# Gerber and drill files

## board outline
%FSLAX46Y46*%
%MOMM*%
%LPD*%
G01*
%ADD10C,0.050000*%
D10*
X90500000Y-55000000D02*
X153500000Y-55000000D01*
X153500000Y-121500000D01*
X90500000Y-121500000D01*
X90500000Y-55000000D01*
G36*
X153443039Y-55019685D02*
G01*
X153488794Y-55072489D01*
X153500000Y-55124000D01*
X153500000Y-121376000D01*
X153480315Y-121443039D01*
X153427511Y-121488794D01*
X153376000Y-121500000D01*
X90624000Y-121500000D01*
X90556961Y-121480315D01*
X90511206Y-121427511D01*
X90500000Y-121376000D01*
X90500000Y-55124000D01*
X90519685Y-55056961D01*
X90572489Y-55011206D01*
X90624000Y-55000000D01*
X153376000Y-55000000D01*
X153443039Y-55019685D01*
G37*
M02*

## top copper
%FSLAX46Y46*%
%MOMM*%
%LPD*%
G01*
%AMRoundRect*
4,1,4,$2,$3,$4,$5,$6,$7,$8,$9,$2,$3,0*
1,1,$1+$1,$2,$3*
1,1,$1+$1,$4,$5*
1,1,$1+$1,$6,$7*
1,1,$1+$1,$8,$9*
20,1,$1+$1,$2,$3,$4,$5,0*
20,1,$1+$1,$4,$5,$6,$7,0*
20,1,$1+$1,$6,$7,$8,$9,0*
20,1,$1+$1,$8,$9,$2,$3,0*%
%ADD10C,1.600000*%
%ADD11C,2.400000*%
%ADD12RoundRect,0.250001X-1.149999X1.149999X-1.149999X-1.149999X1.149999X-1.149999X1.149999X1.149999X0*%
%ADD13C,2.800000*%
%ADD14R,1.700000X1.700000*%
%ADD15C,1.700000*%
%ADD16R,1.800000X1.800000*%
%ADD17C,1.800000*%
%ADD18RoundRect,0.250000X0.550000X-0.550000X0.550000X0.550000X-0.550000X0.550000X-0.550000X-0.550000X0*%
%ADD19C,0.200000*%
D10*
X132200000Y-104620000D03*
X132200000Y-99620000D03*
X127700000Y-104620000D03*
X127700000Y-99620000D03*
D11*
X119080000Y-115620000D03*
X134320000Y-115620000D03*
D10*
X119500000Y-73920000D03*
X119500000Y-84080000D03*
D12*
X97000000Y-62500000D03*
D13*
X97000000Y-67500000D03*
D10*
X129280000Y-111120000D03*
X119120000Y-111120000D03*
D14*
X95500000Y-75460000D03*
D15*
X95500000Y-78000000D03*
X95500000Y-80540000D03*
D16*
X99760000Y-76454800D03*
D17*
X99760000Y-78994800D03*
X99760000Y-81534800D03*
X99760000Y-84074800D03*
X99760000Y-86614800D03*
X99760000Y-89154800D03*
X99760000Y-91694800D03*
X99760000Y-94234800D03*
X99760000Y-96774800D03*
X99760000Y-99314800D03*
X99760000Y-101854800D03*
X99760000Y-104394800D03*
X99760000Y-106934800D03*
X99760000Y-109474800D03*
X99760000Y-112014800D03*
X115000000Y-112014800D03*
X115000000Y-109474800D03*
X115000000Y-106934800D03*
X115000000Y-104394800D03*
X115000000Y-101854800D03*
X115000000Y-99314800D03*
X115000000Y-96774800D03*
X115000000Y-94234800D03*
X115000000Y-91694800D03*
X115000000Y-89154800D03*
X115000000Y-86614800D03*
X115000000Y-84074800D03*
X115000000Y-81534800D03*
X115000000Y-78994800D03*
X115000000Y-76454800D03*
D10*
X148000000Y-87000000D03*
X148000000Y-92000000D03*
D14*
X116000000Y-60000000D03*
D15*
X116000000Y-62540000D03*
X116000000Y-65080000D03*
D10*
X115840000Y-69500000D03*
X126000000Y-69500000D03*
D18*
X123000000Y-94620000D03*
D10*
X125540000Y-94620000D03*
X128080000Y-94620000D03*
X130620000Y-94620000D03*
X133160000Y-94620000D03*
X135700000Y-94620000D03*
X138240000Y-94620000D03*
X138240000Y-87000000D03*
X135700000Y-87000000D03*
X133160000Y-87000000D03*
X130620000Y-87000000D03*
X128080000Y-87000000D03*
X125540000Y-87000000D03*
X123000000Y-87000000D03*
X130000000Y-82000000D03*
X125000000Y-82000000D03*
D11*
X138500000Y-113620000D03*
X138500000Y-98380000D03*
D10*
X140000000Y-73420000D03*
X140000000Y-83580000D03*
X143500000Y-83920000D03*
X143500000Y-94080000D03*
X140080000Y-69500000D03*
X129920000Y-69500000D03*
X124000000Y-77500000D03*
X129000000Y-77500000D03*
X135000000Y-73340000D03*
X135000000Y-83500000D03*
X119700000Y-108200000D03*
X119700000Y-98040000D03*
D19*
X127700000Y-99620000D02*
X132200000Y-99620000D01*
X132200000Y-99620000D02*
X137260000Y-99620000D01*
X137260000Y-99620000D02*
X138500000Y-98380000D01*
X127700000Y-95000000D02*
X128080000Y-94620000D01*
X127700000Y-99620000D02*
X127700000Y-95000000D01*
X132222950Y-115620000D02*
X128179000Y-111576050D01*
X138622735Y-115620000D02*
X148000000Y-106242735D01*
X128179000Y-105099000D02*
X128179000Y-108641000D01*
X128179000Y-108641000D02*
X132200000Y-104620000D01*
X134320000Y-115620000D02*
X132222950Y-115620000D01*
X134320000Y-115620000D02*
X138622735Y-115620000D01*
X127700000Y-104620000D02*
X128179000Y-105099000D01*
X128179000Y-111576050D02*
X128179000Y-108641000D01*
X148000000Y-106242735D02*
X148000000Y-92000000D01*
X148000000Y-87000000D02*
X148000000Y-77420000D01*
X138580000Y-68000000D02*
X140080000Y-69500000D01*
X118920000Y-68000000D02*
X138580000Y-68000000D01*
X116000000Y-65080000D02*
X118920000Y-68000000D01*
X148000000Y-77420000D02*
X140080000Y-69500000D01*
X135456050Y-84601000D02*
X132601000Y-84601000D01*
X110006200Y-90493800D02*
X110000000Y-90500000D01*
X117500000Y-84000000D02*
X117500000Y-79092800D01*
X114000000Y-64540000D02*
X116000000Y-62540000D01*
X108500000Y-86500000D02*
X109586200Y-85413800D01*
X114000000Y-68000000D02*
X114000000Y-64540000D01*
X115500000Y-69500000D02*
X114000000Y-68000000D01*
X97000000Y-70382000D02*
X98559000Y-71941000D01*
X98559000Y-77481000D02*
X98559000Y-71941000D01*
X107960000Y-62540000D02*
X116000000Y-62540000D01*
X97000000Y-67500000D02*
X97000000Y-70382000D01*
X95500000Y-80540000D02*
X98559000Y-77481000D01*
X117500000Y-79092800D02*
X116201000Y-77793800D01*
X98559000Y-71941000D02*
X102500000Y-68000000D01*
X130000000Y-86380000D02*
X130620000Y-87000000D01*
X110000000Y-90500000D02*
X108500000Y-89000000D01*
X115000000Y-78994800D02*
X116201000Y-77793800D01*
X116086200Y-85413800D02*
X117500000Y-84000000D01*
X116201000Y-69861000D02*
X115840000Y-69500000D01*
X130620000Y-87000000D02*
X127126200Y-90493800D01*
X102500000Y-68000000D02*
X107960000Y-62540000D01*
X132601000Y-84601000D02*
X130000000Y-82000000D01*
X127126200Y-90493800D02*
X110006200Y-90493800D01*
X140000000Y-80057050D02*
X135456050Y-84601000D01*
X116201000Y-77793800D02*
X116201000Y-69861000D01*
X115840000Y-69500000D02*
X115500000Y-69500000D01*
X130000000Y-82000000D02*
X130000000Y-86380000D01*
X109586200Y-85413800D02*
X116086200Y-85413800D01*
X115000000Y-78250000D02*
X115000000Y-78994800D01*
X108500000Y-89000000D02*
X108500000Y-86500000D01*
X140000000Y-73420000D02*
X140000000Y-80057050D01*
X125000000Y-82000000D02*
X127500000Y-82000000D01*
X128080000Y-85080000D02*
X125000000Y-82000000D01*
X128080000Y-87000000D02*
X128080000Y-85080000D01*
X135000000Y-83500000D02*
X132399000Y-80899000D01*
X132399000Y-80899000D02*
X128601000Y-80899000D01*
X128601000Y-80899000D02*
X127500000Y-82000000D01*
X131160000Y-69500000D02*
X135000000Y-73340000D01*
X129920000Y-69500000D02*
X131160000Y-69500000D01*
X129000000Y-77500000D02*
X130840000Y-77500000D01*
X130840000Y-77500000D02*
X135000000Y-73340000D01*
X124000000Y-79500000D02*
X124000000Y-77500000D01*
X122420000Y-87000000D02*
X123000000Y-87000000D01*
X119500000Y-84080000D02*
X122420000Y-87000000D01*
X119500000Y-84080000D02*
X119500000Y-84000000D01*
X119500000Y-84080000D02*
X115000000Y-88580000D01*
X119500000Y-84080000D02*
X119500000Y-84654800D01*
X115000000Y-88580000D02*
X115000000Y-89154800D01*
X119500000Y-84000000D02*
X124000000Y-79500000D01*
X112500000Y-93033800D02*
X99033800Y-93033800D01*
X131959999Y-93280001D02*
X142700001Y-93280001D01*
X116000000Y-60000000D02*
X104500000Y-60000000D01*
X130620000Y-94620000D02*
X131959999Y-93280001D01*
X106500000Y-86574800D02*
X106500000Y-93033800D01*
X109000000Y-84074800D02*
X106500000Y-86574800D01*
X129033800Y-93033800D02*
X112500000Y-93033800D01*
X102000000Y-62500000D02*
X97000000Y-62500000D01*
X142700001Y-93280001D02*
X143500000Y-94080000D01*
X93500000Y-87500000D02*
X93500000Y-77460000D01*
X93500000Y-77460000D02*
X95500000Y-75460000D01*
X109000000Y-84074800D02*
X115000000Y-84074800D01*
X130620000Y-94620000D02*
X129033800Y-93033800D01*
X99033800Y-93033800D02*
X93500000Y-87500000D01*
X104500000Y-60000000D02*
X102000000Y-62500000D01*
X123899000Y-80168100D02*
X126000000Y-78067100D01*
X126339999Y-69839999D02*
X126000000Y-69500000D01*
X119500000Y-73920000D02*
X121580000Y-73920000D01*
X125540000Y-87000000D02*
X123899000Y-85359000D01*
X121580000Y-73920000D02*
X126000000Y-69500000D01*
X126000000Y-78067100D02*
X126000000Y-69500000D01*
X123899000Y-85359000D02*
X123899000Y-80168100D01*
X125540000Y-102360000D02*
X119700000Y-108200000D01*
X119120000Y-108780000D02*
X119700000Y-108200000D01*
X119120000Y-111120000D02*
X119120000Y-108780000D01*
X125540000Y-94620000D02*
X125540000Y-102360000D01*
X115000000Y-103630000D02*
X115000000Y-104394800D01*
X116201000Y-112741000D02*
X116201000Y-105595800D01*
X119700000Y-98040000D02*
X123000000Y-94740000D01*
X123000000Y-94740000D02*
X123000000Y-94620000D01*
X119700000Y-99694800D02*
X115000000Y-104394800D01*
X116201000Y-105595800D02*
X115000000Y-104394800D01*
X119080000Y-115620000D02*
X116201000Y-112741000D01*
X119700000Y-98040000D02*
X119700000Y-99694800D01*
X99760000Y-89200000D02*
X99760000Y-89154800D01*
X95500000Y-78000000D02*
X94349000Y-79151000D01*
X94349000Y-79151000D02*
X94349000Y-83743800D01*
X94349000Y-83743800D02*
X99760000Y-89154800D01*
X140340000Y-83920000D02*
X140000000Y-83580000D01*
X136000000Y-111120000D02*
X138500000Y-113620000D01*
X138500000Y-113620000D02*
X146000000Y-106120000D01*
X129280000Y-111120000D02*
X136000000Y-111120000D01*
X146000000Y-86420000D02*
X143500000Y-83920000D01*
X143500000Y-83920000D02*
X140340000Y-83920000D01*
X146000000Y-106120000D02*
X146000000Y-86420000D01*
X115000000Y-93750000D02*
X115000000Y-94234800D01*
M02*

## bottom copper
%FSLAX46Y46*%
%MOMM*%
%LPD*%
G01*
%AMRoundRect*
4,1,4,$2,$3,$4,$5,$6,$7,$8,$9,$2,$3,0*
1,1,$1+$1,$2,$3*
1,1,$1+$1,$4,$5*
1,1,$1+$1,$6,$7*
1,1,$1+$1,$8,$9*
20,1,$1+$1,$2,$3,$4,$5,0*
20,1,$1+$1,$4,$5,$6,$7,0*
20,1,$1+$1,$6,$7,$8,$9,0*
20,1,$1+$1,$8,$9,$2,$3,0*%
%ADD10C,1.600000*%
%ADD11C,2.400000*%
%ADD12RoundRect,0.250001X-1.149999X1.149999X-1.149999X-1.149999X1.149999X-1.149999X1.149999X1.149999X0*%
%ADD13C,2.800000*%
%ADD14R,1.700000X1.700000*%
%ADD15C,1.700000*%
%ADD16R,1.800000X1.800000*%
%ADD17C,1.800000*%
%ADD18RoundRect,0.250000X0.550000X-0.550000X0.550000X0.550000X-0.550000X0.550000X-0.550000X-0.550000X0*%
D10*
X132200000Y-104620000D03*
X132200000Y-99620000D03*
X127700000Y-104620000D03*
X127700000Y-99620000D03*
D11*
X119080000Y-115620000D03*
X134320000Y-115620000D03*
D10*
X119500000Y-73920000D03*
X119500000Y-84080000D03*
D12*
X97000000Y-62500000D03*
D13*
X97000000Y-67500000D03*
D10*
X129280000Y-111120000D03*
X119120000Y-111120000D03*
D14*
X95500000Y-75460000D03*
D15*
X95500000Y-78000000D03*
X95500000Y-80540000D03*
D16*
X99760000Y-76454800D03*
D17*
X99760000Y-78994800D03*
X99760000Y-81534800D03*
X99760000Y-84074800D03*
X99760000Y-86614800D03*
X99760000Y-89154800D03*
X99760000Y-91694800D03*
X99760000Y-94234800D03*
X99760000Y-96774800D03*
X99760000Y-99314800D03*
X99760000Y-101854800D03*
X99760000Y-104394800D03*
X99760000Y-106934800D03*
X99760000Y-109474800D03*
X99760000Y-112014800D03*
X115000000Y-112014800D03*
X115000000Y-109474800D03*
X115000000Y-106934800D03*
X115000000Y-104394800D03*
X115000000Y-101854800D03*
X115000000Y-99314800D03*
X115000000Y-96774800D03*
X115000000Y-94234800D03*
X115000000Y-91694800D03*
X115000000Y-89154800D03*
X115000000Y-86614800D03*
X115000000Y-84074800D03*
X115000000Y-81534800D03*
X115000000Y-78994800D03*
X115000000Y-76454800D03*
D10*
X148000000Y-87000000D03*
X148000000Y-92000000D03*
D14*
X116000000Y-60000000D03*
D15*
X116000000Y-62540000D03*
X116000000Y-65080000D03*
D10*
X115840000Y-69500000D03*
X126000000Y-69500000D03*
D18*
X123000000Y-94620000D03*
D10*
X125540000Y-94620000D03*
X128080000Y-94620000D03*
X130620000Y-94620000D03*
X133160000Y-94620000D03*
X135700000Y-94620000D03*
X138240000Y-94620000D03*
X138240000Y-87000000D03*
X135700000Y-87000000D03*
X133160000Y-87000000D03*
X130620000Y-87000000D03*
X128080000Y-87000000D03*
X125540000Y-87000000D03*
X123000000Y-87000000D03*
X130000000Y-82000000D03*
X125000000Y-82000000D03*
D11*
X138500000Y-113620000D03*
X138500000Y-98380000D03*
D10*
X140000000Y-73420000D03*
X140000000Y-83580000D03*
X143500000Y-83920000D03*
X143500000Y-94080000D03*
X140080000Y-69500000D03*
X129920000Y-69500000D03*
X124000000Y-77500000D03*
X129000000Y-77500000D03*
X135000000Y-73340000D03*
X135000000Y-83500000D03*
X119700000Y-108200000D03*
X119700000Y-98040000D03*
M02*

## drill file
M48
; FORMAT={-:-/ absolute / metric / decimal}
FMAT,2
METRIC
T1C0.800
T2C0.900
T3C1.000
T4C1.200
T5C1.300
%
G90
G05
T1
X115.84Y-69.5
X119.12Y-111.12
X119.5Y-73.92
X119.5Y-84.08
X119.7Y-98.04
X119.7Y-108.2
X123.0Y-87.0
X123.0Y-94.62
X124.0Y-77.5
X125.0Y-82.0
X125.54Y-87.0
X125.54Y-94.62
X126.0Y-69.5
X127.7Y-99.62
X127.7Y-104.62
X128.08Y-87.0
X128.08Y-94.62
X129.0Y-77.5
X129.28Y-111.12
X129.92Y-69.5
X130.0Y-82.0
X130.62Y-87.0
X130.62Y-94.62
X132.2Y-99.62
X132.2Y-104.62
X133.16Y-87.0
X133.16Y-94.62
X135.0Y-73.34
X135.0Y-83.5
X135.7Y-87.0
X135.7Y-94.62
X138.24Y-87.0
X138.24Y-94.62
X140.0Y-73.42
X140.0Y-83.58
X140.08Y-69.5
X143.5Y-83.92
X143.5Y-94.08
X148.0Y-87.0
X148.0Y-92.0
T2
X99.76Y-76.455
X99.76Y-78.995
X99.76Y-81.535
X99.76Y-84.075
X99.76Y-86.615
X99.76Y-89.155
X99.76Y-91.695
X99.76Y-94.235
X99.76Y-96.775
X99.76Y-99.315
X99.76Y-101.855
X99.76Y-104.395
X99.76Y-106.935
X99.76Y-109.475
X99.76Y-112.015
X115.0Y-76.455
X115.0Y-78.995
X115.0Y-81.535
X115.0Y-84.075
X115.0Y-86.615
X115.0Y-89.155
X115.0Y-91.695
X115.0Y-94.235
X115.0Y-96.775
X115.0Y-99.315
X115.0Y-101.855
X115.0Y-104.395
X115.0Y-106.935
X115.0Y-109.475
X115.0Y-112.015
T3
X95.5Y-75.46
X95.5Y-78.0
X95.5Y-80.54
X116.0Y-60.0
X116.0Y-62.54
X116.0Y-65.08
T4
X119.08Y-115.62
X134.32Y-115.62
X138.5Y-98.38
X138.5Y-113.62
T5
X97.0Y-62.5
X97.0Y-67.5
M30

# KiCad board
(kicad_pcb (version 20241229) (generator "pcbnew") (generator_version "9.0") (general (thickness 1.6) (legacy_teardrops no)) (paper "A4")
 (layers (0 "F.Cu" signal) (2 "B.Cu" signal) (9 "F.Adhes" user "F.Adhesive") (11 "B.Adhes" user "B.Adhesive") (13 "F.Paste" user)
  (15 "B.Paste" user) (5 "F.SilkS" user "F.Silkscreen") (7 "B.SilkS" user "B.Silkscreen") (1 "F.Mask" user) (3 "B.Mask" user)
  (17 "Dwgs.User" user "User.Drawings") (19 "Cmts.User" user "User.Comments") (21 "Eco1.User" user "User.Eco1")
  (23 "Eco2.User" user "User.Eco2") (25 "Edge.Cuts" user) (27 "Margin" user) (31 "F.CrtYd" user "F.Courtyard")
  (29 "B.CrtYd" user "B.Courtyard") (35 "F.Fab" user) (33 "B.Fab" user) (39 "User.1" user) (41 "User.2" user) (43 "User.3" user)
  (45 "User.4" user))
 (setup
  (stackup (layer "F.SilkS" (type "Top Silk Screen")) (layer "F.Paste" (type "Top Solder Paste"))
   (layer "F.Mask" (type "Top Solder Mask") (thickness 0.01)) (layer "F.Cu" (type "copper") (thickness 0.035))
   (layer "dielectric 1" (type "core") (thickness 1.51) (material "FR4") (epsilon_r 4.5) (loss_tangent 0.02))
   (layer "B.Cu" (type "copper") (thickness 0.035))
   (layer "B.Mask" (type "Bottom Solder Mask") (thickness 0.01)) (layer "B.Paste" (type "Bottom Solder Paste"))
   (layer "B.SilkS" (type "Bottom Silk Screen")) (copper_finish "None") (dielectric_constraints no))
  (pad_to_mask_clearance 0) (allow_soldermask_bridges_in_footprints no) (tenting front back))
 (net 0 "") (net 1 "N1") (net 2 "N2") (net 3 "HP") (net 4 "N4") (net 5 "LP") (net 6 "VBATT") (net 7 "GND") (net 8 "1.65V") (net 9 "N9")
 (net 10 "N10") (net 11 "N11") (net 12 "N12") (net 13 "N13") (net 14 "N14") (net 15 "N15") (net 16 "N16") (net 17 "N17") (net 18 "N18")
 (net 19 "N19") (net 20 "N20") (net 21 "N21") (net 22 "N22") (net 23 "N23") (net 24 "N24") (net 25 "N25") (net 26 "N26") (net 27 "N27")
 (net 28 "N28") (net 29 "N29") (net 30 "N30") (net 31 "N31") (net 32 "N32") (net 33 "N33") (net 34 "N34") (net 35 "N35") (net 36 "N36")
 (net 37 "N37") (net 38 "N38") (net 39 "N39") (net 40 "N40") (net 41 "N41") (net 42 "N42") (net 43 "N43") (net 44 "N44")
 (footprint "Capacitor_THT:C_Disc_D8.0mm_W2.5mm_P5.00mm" (layer "F.Cu") (at 132.2 104.62 90)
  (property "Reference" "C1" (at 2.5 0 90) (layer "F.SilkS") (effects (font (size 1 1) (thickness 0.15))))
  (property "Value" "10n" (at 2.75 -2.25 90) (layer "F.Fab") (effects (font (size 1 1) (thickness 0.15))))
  (pad "1" thru_hole circle (at 0 0 90) (size 1.6 1.6) (drill 0.8) (layers "*.Cu" "*.Mask") (remove_unused_layers no) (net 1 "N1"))
  (pad "2" thru_hole circle (at 5 0 90) (size 1.6 1.6) (drill 0.8) (layers "*.Cu" "*.Mask") (remove_unused_layers no) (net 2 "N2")))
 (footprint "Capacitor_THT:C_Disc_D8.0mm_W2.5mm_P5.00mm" (layer "F.Cu") (at 127.7 104.62 90)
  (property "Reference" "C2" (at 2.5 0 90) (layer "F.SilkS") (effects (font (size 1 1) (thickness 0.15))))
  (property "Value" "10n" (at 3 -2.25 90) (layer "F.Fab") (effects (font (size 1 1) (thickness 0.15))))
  (pad "1" thru_hole circle (at 0 0 90) (size 1.6 1.6) (drill 0.8) (layers "*.Cu" "*.Mask") (remove_unused_layers no) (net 1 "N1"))
  (pad "2" thru_hole circle (at 5 0 90) (size 1.6 1.6) (drill 0.8) (layers "*.Cu" "*.Mask") (remove_unused_layers no) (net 2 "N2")))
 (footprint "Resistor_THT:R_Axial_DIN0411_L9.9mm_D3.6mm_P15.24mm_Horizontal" (layer "F.Cu") (at 119.08 115.62)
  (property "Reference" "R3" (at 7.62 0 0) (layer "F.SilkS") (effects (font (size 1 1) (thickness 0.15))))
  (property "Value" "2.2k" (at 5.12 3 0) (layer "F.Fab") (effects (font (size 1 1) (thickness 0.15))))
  (pad "1" thru_hole circle (at 0 0) (size 2.4 2.4) (drill 1.2) (layers "*.Cu" "*.Mask") (remove_unused_layers no) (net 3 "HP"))
  (pad "2" thru_hole circle (at 15.24 0) (size 2.4 2.4) (drill 1.2) (layers "*.Cu" "*.Mask") (remove_unused_layers no) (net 1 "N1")))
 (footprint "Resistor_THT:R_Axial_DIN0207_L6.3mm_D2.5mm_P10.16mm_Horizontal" (layer "F.Cu") (at 119.5 73.92 -90)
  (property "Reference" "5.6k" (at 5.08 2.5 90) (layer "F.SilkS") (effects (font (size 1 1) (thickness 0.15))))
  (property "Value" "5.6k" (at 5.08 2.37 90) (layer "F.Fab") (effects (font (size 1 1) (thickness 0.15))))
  (pad "1" thru_hole circle (at 0 0 270) (size 1.6 1.6) (drill 0.8) (layers "*.Cu" "*.Mask") (remove_unused_layers no) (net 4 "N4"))
  (pad "2" thru_hole circle (at 10.16 0 270) (size 1.6 1.6) (drill 0.8) (layers "*.Cu" "*.Mask") (remove_unused_layers no) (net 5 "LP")))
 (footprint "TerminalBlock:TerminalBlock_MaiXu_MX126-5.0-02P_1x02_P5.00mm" (layer "F.Cu") (at 97 62.5 -90)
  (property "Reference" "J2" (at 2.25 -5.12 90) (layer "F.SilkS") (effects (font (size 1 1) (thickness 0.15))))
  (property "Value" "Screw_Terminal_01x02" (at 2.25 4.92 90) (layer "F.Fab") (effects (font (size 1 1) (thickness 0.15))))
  (pad "1" thru_hole roundrect (at 0 0 270) (size 2.8 2.8) (drill 1.3) (layers "*.Cu" "*.Mask") (remove_unused_layers no)
   (roundrect_rratio 0.089286) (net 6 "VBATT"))
  (pad "2" thru_hole circle (at 5 0 270) (size 2.8 2.8) (drill 1.3) (layers "*.Cu" "*.Mask") (remove_unused_layers no) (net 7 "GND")))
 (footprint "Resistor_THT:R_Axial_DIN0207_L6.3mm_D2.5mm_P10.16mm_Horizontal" (layer "F.Cu") (at 129.28 111.12 180)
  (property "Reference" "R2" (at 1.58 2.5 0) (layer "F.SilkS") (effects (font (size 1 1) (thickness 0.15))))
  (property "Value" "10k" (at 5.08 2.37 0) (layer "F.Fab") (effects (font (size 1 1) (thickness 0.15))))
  (pad "1" thru_hole circle (at 0 0 180) (size 1.6 1.6) (drill 0.8) (layers "*.Cu" "*.Mask") (remove_unused_layers no) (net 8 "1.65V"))
  (pad "2" thru_hole circle (at 10.16 0 180) (size 1.6 1.6) (drill 0.8) (layers "*.Cu" "*.Mask") (remove_unused_layers no) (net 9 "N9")))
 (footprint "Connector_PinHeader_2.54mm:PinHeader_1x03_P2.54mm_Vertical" (layer "F.Cu") (at 95.5 75.46)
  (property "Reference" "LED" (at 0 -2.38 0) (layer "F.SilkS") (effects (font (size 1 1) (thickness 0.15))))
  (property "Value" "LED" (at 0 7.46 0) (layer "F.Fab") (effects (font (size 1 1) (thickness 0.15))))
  (pad "1" thru_hole rect (at 0 0) (size 1.7 1.7) (drill 1) (layers "*.Cu" "*.Mask") (remove_unused_layers no) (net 6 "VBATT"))
  (pad "2" thru_hole circle (at 0 2.54) (size 1.7 1.7) (drill 1) (layers "*.Cu" "*.Mask") (remove_unused_layers no) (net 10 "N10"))
  (pad "3" thru_hole circle (at 0 5.08) (size 1.7 1.7) (drill 1) (layers "*.Cu" "*.Mask") (remove_unused_layers no) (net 7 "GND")))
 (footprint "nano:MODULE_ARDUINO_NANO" (layer "F.Cu") (at 107.38 94.2348)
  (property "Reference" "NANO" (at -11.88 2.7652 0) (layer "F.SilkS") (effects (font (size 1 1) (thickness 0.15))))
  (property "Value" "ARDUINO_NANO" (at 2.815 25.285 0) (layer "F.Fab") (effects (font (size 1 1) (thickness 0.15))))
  (pad "1" thru_hole rect (at -7.62 -17.78) (size 1.8 1.8) (drill 0.9) (layers "*.Cu" "*.Mask") (remove_unused_layers no) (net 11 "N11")
   (solder_mask_margin 0.102))
  (pad "2" thru_hole circle (at -7.62 -15.24) (size 1.8 1.8) (drill 0.9) (layers "*.Cu" "*.Mask") (remove_unused_layers no) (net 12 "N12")
   (solder_mask_margin 0.102))
  (pad "3" thru_hole circle (at -7.62 -12.7) (size 1.8 1.8) (drill 0.9) (layers "*.Cu" "*.Mask") (remove_unused_layers no) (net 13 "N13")
   (solder_mask_margin 0.102))
  (pad "4" thru_hole circle (at -7.62 -10.16) (size 1.8 1.8) (drill 0.9) (layers "*.Cu" "*.Mask") (remove_unused_layers no) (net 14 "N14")
   (solder_mask_margin 0.102))
  (pad "5" thru_hole circle (at -7.62 -7.62) (size 1.8 1.8) (drill 0.9) (layers "*.Cu" "*.Mask") (remove_unused_layers no) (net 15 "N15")
   (solder_mask_margin 0.102))
  (pad "6" thru_hole circle (at -7.62 -5.08) (size 1.8 1.8) (drill 0.9) (layers "*.Cu" "*.Mask") (remove_unused_layers no) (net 10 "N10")
   (solder_mask_margin 0.102))
  (pad "7" thru_hole circle (at -7.62 -2.54) (size 1.8 1.8) (drill 0.9) (layers "*.Cu" "*.Mask") (remove_unused_layers no) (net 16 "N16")
   (solder_mask_margin 0.102))
  (pad "8" thru_hole circle (at -7.62 0) (size 1.8 1.8) (drill 0.9) (layers "*.Cu" "*.Mask") (remove_unused_layers no) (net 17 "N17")
   (solder_mask_margin 0.102))
  (pad "9" thru_hole circle (at -7.62 2.54) (size 1.8 1.8) (drill 0.9) (layers "*.Cu" "*.Mask") (remove_unused_layers no) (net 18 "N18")
   (solder_mask_margin 0.102))
  (pad "10" thru_hole circle (at -7.62 5.08) (size 1.8 1.8) (drill 0.9) (layers "*.Cu" "*.Mask") (remove_unused_layers no) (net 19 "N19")
   (solder_mask_margin 0.102))
  (pad "11" thru_hole circle (at -7.62 7.62) (size 1.8 1.8) (drill 0.9) (layers "*.Cu" "*.Mask") (remove_unused_layers no) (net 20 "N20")
   (solder_mask_margin 0.102))
  (pad "12" thru_hole circle (at -7.62 10.16) (size 1.8 1.8) (drill 0.9) (layers "*.Cu" "*.Mask") (remove_unused_layers no) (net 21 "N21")
   (solder_mask_margin 0.102))
  (pad "13" thru_hole circle (at -7.62 12.7) (size 1.8 1.8) (drill 0.9) (layers "*.Cu" "*.Mask") (remove_unused_layers no) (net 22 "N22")
   (solder_mask_margin 0.102))
  (pad "14" thru_hole circle (at -7.62 15.24) (size 1.8 1.8) (drill 0.9) (layers "*.Cu" "*.Mask") (remove_unused_layers no) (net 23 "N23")
   (solder_mask_margin 0.102))
  (pad "15" thru_hole circle (at -7.62 17.78) (size 1.8 1.8) (drill 0.9) (layers "*.Cu" "*.Mask") (remove_unused_layers no) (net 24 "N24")
   (solder_mask_margin 0.102))
  (pad "16" thru_hole circle (at 7.62 17.78) (size 1.8 1.8) (drill 0.9) (layers "*.Cu" "*.Mask") (remove_unused_layers no) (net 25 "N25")
   (solder_mask_margin 0.102))
  (pad "17" thru_hole circle (at 7.62 15.24) (size 1.8 1.8) (drill 0.9) (layers "*.Cu" "*.Mask") (remove_unused_layers no) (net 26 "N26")
   (solder_mask_margin 0.102))
  (pad "18" thru_hole circle (at 7.62 12.7) (size 1.8 1.8) (drill 0.9) (layers "*.Cu" "*.Mask") (remove_unused_layers no) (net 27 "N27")
   (solder_mask_margin 0.102))
  (pad "19" thru_hole circle (at 7.62 10.16) (size 1.8 1.8) (drill 0.9) (layers "*.Cu" "*.Mask") (remove_unused_layers no) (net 3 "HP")
   (solder_mask_margin 0.102))
  (pad "20" thru_hole circle (at 7.62 7.62) (size 1.8 1.8) (drill 0.9) (layers "*.Cu" "*.Mask") (remove_unused_layers no) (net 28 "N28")
   (solder_mask_margin 0.102))
  (pad "21" thru_hole circle (at 7.62 5.08) (size 1.8 1.8) (drill 0.9) (layers "*.Cu" "*.Mask") (remove_unused_layers no) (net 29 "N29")
   (solder_mask_margin 0.102))
  (pad "22" thru_hole circle (at 7.62 2.54) (size 1.8 1.8) (drill 0.9) (layers "*.Cu" "*.Mask") (remove_unused_layers no) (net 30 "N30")
   (solder_mask_margin 0.102))
  (pad "23" thru_hole circle (at 7.62 0) (size 1.8 1.8) (drill 0.9) (layers "*.Cu" "*.Mask") (remove_unused_layers no) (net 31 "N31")
   (solder_mask_margin 0.102))
  (pad "24" thru_hole circle (at 7.62 -2.54) (size 1.8 1.8) (drill 0.9) (layers "*.Cu" "*.Mask") (remove_unused_layers no) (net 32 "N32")
   (solder_mask_margin 0.102))
  (pad "25" thru_hole circle (at 7.62 -5.08) (size 1.8 1.8) (drill 0.9) (layers "*.Cu" "*.Mask") (remove_unused_layers no) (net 5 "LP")
   (solder_mask_margin 0.102))
  (pad "26" thru_hole circle (at 7.62 -7.62) (size 1.8 1.8) (drill 0.9) (layers "*.Cu" "*.Mask") (remove_unused_layers no) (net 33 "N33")
   (solder_mask_margin 0.102))
  (pad "27" thru_hole circle (at 7.62 -10.16) (size 1.8 1.8) (drill 0.9) (layers "*.Cu" "*.Mask") (remove_unused_layers no) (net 6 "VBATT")
   (solder_mask_margin 0.102))
  (pad "28" thru_hole circle (at 7.62 -12.7) (size 1.8 1.8) (drill 0.9) (layers "*.Cu" "*.Mask") (remove_unused_layers no) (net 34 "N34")
   (solder_mask_margin 0.102))
  (pad "29" thru_hole circle (at 7.62 -15.24) (size 1.8 1.8) (drill 0.9) (layers "*.Cu" "*.Mask") (remove_unused_layers no) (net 7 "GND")
   (solder_mask_margin 0.102))
  (pad "30" thru_hole circle (at 7.62 -17.78) (size 1.8 1.8) (drill 0.9) (layers "*.Cu" "*.Mask") (remove_unused_layers no) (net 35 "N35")
   (solder_mask_margin 0.102)))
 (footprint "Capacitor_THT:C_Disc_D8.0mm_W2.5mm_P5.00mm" (layer "F.Cu") (at 148 87 -90)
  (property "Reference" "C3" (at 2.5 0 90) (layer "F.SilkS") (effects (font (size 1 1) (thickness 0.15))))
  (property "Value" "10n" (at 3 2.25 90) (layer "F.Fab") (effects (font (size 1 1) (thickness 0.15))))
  (pad "1" thru_hole circle (at 0 0 270) (size 1.6 1.6) (drill 0.8) (layers "*.Cu" "*.Mask") (remove_unused_layers no) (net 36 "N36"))
  (pad "2" thru_hole circle (at 5 0 270) (size 1.6 1.6) (drill 0.8) (layers "*.Cu" "*.Mask") (remove_unused_layers no) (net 1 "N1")))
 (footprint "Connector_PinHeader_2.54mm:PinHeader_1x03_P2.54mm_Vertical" (layer "F.Cu") (at 116 60)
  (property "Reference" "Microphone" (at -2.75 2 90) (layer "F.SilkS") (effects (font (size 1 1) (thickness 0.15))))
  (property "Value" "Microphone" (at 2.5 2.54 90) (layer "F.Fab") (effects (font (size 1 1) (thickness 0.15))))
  (pad "1" thru_hole rect (at 0 0) (size 1.7 1.7) (drill 1) (layers "*.Cu" "*.Mask") (remove_unused_layers no) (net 6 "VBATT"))
  (pad "2" thru_hole circle (at 0 2.54) (size 1.7 1.7) (drill 1) (layers "*.Cu" "*.Mask") (remove_unused_layers no) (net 7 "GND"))
  (pad "3" thru_hole circle (at 0 5.08) (size 1.7 1.7) (drill 1) (layers "*.Cu" "*.Mask") (remove_unused_layers no) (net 36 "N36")))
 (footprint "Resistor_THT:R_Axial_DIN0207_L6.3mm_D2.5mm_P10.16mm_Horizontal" (layer "F.Cu") (at 115.84 69.5)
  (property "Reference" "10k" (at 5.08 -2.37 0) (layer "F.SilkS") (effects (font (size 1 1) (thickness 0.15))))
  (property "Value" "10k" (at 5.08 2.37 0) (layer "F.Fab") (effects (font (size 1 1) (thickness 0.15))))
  (pad "1" thru_hole circle (at 0 0) (size 1.6 1.6) (drill 0.8) (layers "*.Cu" "*.Mask") (remove_unused_layers no) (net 7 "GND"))
  (pad "2" thru_hole circle (at 10.16 0) (size 1.6 1.6) (drill 0.8) (layers "*.Cu" "*.Mask") (remove_unused_layers no) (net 4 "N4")))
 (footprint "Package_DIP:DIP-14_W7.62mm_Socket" (layer "F.Cu") (at 123 94.62 90)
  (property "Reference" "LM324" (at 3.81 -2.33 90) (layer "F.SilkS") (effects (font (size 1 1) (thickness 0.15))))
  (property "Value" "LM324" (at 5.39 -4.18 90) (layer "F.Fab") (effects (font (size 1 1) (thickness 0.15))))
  (pad "1" thru_hole roundrect (at 0 0 90) (size 1.6 1.6) (drill 0.8) (layers "*.Cu" "*.Mask") (remove_unused_layers no)
   (roundrect_rratio 0.15625) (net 3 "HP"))
  (pad "2" thru_hole circle (at 0 2.54 90) (size 1.6 1.6) (drill 0.8) (layers "*.Cu" "*.Mask") (remove_unused_layers no) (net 9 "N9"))
  (pad "3" thru_hole circle (at 0 5.08 90) (size 1.6 1.6) (drill 0.8) (layers "*.Cu" "*.Mask") (remove_unused_layers no) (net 2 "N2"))
  (pad "4" thru_hole circle (at 0 7.62 90) (size 1.6 1.6) (drill 0.8) (layers "*.Cu" "*.Mask") (remove_unused_layers no) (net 6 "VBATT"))
  (pad "5" thru_hole circle (at 0 10.16 90) (size 1.6 1.6) (drill 0.8) (layers "*.Cu" "*.Mask") (remove_unused_layers no) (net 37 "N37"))
  (pad "6" thru_hole circle (at 0 12.7 90) (size 1.6 1.6) (drill 0.8) (layers "*.Cu" "*.Mask") (remove_unused_layers no) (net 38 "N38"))
  (pad "7" thru_hole circle (at 0 15.24 90) (size 1.6 1.6) (drill 0.8) (layers "*.Cu" "*.Mask") (remove_unused_layers no) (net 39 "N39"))
  (pad "8" thru_hole circle (at 7.62 15.24 90) (size 1.6 1.6) (drill 0.8) (layers "*.Cu" "*.Mask") (remove_unused_layers no) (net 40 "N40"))
  (pad "9" thru_hole circle (at 7.62 12.7 90) (size 1.6 1.6) (drill 0.8) (layers "*.Cu" "*.Mask") (remove_unused_layers no) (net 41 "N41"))
  (pad "10" thru_hole circle (at 7.62 10.16 90) (size 1.6 1.6) (drill 0.8) (layers "*.Cu" "*.Mask") (remove_unused_layers no) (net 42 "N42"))
  (pad "11" thru_hole circle (at 7.62 7.62 90) (size 1.6 1.6) (drill 0.8) (layers "*.Cu" "*.Mask") (remove_unused_layers no) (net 7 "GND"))
  (pad "12" thru_hole circle (at 7.62 5.08 90) (size 1.6 1.6) (drill 0.8) (layers "*.Cu" "*.Mask") (remove_unused_layers no) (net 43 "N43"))
  (pad "13" thru_hole circle (at 7.62 2.54 90) (size 1.6 1.6) (drill 0.8) (layers "*.Cu" "*.Mask") (remove_unused_layers no) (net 4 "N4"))
  (pad "14" thru_hole circle (at 7.62 0 90) (size 1.6 1.6) (drill 0.8) (layers "*.Cu" "*.Mask") (remove_unused_layers no) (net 5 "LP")))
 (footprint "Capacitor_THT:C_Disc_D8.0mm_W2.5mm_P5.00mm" (layer "F.Cu") (at 130 82 180)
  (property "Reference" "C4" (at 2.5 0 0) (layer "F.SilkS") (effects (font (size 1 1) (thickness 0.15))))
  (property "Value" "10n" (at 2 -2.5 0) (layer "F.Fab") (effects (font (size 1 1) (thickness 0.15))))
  (pad "1" thru_hole circle (at 0 0 180) (size 1.6 1.6) (drill 0.8) (layers "*.Cu" "*.Mask") (remove_unused_layers no) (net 7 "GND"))
  (pad "2" thru_hole circle (at 5 0 180) (size 1.6 1.6) (drill 0.8) (layers "*.Cu" "*.Mask") (remove_unused_layers no) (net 43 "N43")))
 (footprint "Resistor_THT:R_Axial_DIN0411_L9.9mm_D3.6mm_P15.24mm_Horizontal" (layer "F.Cu") (at 138.5 113.62 90)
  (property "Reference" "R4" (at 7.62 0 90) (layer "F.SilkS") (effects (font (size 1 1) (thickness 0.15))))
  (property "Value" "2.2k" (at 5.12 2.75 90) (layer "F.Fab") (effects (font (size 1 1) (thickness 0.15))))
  (pad "1" thru_hole circle (at 0 0 90) (size 2.4 2.4) (drill 1.2) (layers "*.Cu" "*.Mask") (remove_unused_layers no) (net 8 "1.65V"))
  (pad "2" thru_hole circle (at 15.24 0 90) (size 2.4 2.4) (drill 1.2) (layers "*.Cu" "*.Mask") (remove_unused_layers no) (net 2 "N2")))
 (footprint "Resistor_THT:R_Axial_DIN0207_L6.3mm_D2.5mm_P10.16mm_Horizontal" (layer "F.Cu") (at 140 73.42 -90)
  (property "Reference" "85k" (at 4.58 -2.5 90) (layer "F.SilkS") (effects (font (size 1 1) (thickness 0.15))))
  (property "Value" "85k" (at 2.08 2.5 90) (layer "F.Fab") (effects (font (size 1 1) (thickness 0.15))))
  (pad "1" thru_hole circle (at 0 0 270) (size 1.6 1.6) (drill 0.8) (layers "*.Cu" "*.Mask") (remove_unused_layers no) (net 7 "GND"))
  (pad "2" thru_hole circle (at 10.16 0 270) (size 1.6 1.6) (drill 0.8) (layers "*.Cu" "*.Mask") (remove_unused_layers no) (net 8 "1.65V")))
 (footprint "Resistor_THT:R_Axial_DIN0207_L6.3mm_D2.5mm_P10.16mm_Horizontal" (layer "F.Cu") (at 143.5 83.92 -90)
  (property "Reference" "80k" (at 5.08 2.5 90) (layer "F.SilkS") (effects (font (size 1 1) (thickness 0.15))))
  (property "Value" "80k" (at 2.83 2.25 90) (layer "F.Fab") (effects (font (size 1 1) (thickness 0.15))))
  (pad "1" thru_hole circle (at 0 0 270) (size 1.6 1.6) (drill 0.8) (layers "*.Cu" "*.Mask") (remove_unused_layers no) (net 8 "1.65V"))
  (pad "2" thru_hole circle (at 10.16 0 270) (size 1.6 1.6) (drill 0.8) (layers "*.Cu" "*.Mask") (remove_unused_layers no) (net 6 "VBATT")))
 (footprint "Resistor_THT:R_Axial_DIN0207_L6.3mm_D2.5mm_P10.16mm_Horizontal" (layer "F.Cu") (at 140.08 69.5 180)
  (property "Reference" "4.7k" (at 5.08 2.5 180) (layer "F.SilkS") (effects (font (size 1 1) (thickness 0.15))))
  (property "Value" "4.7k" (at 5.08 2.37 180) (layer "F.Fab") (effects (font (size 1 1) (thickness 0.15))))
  (pad "1" thru_hole circle (at 0 0 180) (size 1.6 1.6) (drill 0.8) (layers "*.Cu" "*.Mask") (remove_unused_layers no) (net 36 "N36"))
  (pad "2" thru_hole circle (at 10.16 0 180) (size 1.6 1.6) (drill 0.8) (layers "*.Cu" "*.Mask") (remove_unused_layers no) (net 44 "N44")))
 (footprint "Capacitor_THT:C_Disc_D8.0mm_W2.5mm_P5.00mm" (layer "F.Cu") (at 124 77.5)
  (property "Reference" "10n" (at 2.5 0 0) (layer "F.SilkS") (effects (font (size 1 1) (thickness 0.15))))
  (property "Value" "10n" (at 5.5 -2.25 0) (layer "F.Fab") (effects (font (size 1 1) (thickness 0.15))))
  (pad "1" thru_hole circle (at 0 0) (size 1.6 1.6) (drill 0.8) (layers "*.Cu" "*.Mask") (remove_unused_layers no) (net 5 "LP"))
  (pad "2" thru_hole circle (at 5 0) (size 1.6 1.6) (drill 0.8) (layers "*.Cu" "*.Mask") (remove_unused_layers no) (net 44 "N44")))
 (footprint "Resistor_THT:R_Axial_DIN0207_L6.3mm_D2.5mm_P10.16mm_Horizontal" (layer "F.Cu") (at 135 73.34 -90)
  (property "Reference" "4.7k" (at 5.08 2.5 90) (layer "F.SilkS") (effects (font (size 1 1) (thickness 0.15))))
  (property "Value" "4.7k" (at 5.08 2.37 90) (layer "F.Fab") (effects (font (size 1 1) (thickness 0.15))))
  (pad "1" thru_hole circle (at 0 0 270) (size 1.6 1.6) (drill 0.8) (layers "*.Cu" "*.Mask") (remove_unused_layers no) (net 44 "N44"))
  (pad "2" thru_hole circle (at 10.16 0 270) (size 1.6 1.6) (drill 0.8) (layers "*.Cu" "*.Mask") (remove_unused_layers no) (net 43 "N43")))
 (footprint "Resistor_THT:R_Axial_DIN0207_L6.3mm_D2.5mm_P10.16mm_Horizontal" (layer "F.Cu") (at 119.7 108.2 90)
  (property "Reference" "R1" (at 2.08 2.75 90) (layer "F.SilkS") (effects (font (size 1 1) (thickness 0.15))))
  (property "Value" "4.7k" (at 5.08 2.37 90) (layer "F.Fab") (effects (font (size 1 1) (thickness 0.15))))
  (pad "1" thru_hole circle (at 0 0 90) (size 1.6 1.6) (drill 0.8) (layers "*.Cu" "*.Mask") (remove_unused_layers no) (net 9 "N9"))
  (pad "2" thru_hole circle (at 10.16 0 90) (size 1.6 1.6) (drill 0.8) (layers "*.Cu" "*.Mask") (remove_unused_layers no) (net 3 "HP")))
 (gr_rect (start 90.5 55) (end 153.5 121.5) (stroke (width 0.05) (type solid)) (fill no) (layer "Edge.Cuts"))
 (segment (start 127.7 99.62) (end 132.2 99.62) (width 0.2) (layer "F.Cu") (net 2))
 (segment (start 132.2 99.62) (end 137.26 99.62) (width 0.2) (layer "F.Cu") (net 2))
 (segment (start 137.26 99.62) (end 138.5 98.38) (width 0.2) (layer "F.Cu") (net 2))
 (segment (start 127.7 95) (end 128.08 94.62) (width 0.2) (layer "F.Cu") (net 2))
 (segment (start 127.7 99.62) (end 127.7 95) (width 0.2) (layer "F.Cu") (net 2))
 (segment (start 132.22295 115.62) (end 128.179 111.57605) (width 0.2) (layer "F.Cu") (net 1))
 (segment (start 138.622735 115.62) (end 148 106.242735) (width 0.2) (layer "F.Cu") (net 1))
 (segment (start 128.179 105.099) (end 128.179 108.641) (width 0.2) (layer "F.Cu") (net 1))
 (segment (start 128.179 108.641) (end 132.2 104.62) (width 0.2) (layer "F.Cu") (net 1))
 (segment (start 134.32 115.62) (end 132.22295 115.62) (width 0.2) (layer "F.Cu") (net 1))
 (segment (start 134.32 115.62) (end 138.622735 115.62) (width 0.2) (layer "F.Cu") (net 1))
 (segment (start 127.7 104.62) (end 128.179 105.099) (width 0.2) (layer "F.Cu") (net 1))
 (segment (start 128.179 111.57605) (end 128.179 108.641) (width 0.2) (layer "F.Cu") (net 1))
 (segment (start 148 106.242735) (end 148 92) (width 0.2) (layer "F.Cu") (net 1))
 (segment (start 148 87) (end 148 77.42) (width 0.2) (layer "F.Cu") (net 36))
 (segment (start 138.58 68) (end 140.08 69.5) (width 0.2) (layer "F.Cu") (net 36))
 (segment (start 118.92 68) (end 138.58 68) (width 0.2) (layer "F.Cu") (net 36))
 (segment (start 116 65.08) (end 118.92 68) (width 0.2) (layer "F.Cu") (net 36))
 (segment (start 148 77.42) (end 140.08 69.5) (width 0.2) (layer "F.Cu") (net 36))
 (segment (start 135.45605 84.601) (end 132.601 84.601) (width 0.2) (layer "F.Cu") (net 7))
 (segment (start 110.0062 90.4938) (end 110 90.5) (width 0.2) (layer "F.Cu") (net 7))
 (segment (start 117.5 84) (end 117.5 79.0928) (width 0.2) (layer "F.Cu") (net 7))
 (segment (start 114 64.54) (end 116 62.54) (width 0.2) (layer "F.Cu") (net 7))
 (segment (start 108.5 86.5) (end 109.5862 85.4138) (width 0.2) (layer "F.Cu") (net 7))
 (segment (start 114 68) (end 114 64.54) (width 0.2) (layer "F.Cu") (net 7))
 (segment (start 115.5 69.5) (end 114 68) (width 0.2) (layer "F.Cu") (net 7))
 (segment (start 97 70.382) (end 98.559 71.941) (width 0.2) (layer "F.Cu") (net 7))
 (segment (start 98.559 77.481) (end 98.559 71.941) (width 0.2) (layer "F.Cu") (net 7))
 (segment (start 107.96 62.54) (end 116 62.54) (width 0.2) (layer "F.Cu") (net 7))
 (segment (start 97 67.5) (end 97 70.382) (width 0.2) (layer "F.Cu") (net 7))
 (segment (start 95.5 80.54) (end 98.559 77.481) (width 0.2) (layer "F.Cu") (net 7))
 (segment (start 117.5 79.0928) (end 116.201 77.7938) (width 0.2) (layer "F.Cu") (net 7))
 (segment (start 98.559 71.941) (end 102.5 68) (width 0.2) (layer "F.Cu") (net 7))
 (segment (start 130 86.38) (end 130.62 87) (width 0.2) (layer "F.Cu") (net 7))
 (segment (start 110 90.5) (end 108.5 89) (width 0.2) (layer "F.Cu") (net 7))
 (segment (start 115 78.9948) (end 116.201 77.7938) (width 0.2) (layer "F.Cu") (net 7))
 (segment (start 116.0862 85.4138) (end 117.5 84) (width 0.2) (layer "F.Cu") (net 7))
 (segment (start 116.201 69.861) (end 115.84 69.5) (width 0.2) (layer "F.Cu") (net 7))
 (segment (start 130.62 87) (end 127.1262 90.4938) (width 0.2) (layer "F.Cu") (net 7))
 (segment (start 102.5 68) (end 107.96 62.54) (width 0.2) (layer "F.Cu") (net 7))
 (segment (start 132.601 84.601) (end 130 82) (width 0.2) (layer "F.Cu") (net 7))
 (segment (start 127.1262 90.4938) (end 110.0062 90.4938) (width 0.2) (layer "F.Cu") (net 7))
 (segment (start 140 80.05705) (end 135.45605 84.601) (width 0.2) (layer "F.Cu") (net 7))
 (segment (start 116.201 77.7938) (end 116.201 69.861) (width 0.2) (layer "F.Cu") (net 7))
 (segment (start 115.84 69.5) (end 115.5 69.5) (width 0.2) (layer "F.Cu") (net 7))
 (segment (start 130 82) (end 130 86.38) (width 0.2) (layer "F.Cu") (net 7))
 (segment (start 109.5862 85.4138) (end 116.0862 85.4138) (width 0.2) (layer "F.Cu") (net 7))
 (segment (start 115 78.25) (end 115 78.9948) (width 0.2) (layer "F.Cu") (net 7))
 (segment (start 108.5 89) (end 108.5 86.5) (width 0.2) (layer "F.Cu") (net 7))
 (segment (start 140 73.42) (end 140 80.05705) (width 0.2) (layer "F.Cu") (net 7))
 (segment (start 125 82) (end 127.5 82) (width 0.2) (layer "F.Cu") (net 43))
 (segment (start 128.08 85.08) (end 125 82) (width 0.2) (layer "F.Cu") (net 43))
 (segment (start 128.08 87) (end 128.08 85.08) (width 0.2) (layer "F.Cu") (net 43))
 (segment (start 135 83.5) (end 132.399 80.899) (width 0.2) (layer "F.Cu") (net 43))
 (segment (start 132.399 80.899) (end 128.601 80.899) (width 0.2) (layer "F.Cu") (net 43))
 (segment (start 128.601 80.899) (end 127.5 82) (width 0.2) (layer "F.Cu") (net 43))
 (segment (start 131.16 69.5) (end 135 73.34) (width 0.2) (layer "F.Cu") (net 44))
 (segment (start 129.92 69.5) (end 131.16 69.5) (width 0.2) (layer "F.Cu") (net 44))
 (segment (start 129 77.5) (end 130.84 77.5) (width 0.2) (layer "F.Cu") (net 44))
 (segment (start 130.84 77.5) (end 135 73.34) (width 0.2) (layer "F.Cu") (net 44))
 (segment (start 124 79.5) (end 124 77.5) (width 0.2) (layer "F.Cu") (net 5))
 (segment (start 122.42 87) (end 123 87) (width 0.2) (layer "F.Cu") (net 5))
 (segment (start 119.5 84.08) (end 122.42 87) (width 0.2) (layer "F.Cu") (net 5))
 (segment (start 119.5 84.08) (end 119.5 84) (width 0.2) (layer "F.Cu") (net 5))
 (segment (start 119.5 84.08) (end 115 88.58) (width 0.2) (layer "F.Cu") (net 5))
 (segment (start 119.5 84.08) (end 119.5 84.6548) (width 0.2) (layer "F.Cu") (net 5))
 (segment (start 115 88.58) (end 115 89.1548) (width 0.2) (layer "F.Cu") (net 5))
 (segment (start 119.5 84) (end 124 79.5) (width 0.2) (layer "F.Cu") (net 5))
 (segment (start 112.5 93.0338) (end 99.0338 93.0338) (width 0.2) (layer "F.Cu") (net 6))
 (segment (start 131.959999 93.280001) (end 142.700001 93.280001) (width 0.2) (layer "F.Cu") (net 6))
 (segment (start 116 60) (end 104.5 60) (width 0.2) (layer "F.Cu") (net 6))
 (segment (start 130.62 94.62) (end 131.959999 93.280001) (width 0.2) (layer "F.Cu") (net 6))
 (segment (start 106.5 86.5748) (end 106.5 93.0338) (width 0.2) (layer "F.Cu") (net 6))
 (segment (start 109 84.0748) (end 106.5 86.5748) (width 0.2) (layer "F.Cu") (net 6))
 (segment (start 129.0338 93.0338) (end 112.5 93.0338) (width 0.2) (layer "F.Cu") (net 6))
 (segment (start 102 62.5) (end 97 62.5) (width 0.2) (layer "F.Cu") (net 6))
 (segment (start 142.700001 93.280001) (end 143.5 94.08) (width 0.2) (layer "F.Cu") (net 6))
 (segment (start 93.5 87.5) (end 93.5 77.46) (width 0.2) (layer "F.Cu") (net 6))
 (segment (start 93.5 77.46) (end 95.5 75.46) (width 0.2) (layer "F.Cu") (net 6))
 (segment (start 109 84.0748) (end 115 84.0748) (width 0.2) (layer "F.Cu") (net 6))
 (segment (start 130.62 94.62) (end 129.0338 93.0338) (width 0.2) (layer "F.Cu") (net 6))
 (segment (start 99.0338 93.0338) (end 93.5 87.5) (width 0.2) (layer "F.Cu") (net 6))
 (segment (start 104.5 60) (end 102 62.5) (width 0.2) (layer "F.Cu") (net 6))
 (segment (start 123.899 80.1681) (end 126 78.0671) (width 0.2) (layer "F.Cu") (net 4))
 (segment (start 126.339999 69.839999) (end 126 69.5) (width 0.2) (layer "F.Cu") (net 4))
 (segment (start 119.5 73.92) (end 121.58 73.92) (width 0.2) (layer "F.Cu") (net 4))
 (segment (start 125.54 87) (end 123.899 85.359) (width 0.2) (layer "F.Cu") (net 4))
 (segment (start 121.58 73.92) (end 126 69.5) (width 0.2) (layer "F.Cu") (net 4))
 (segment (start 126 78.0671) (end 126 69.5) (width 0.2) (layer "F.Cu") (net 4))
 (segment (start 123.899 85.359) (end 123.899 80.1681) (width 0.2) (layer "F.Cu") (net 4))
 (segment (start 125.54 102.36) (end 119.7 108.2) (width 0.2) (layer "F.Cu") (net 9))
 (segment (start 119.12 108.78) (end 119.7 108.2) (width 0.2) (layer "F.Cu") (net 9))
 (segment (start 119.12 111.12) (end 119.12 108.78) (width 0.2) (layer "F.Cu") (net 9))
 (segment (start 125.54 94.62) (end 125.54 102.36) (width 0.2) (layer "F.Cu") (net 9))
 (segment (start 115 103.63) (end 115 104.3948) (width 0.2) (layer "F.Cu") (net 3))
 (segment (start 116.201 112.741) (end 116.201 105.5958) (width 0.2) (layer "F.Cu") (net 3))
 (segment (start 119.7 98.04) (end 123 94.74) (width 0.2) (layer "F.Cu") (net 3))
 (segment (start 123 94.74) (end 123 94.62) (width 0.2) (layer "F.Cu") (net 3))
 (segment (start 119.7 99.6948) (end 115 104.3948) (width 0.2) (layer "F.Cu") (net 3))
 (segment (start 116.201 105.5958) (end 115 104.3948) (width 0.2) (layer "F.Cu") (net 3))
 (segment (start 119.08 115.62) (end 116.201 112.741) (width 0.2) (layer "F.Cu") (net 3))
 (segment (start 119.7 98.04) (end 119.7 99.6948) (width 0.2) (layer "F.Cu") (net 3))
 (segment (start 99.76 89.2) (end 99.76 89.1548) (width 0.2) (layer "F.Cu") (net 10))
 (segment (start 95.5 78) (end 94.349 79.151) (width 0.2) (layer "F.Cu") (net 10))
 (segment (start 94.349 79.151) (end 94.349 83.7438) (width 0.2) (layer "F.Cu") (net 10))
 (segment (start 94.349 83.7438) (end 99.76 89.1548) (width 0.2) (layer "F.Cu") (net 10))
 (segment (start 140.34 83.92) (end 140 83.58) (width 0.2) (layer "F.Cu") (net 8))
 (segment (start 136 111.12) (end 138.5 113.62) (width 0.2) (layer "F.Cu") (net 8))
 (segment (start 138.5 113.62) (end 146 106.12) (width 0.2) (layer "F.Cu") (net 8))
 (segment (start 129.28 111.12) (end 136 111.12) (width 0.2) (layer "F.Cu") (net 8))
 (segment (start 146 86.42) (end 143.5 83.92) (width 0.2) (layer "F.Cu") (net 8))
 (segment (start 143.5 83.92) (end 140.34 83.92) (width 0.2) (layer "F.Cu") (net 8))
 (segment (start 146 106.12) (end 146 86.42) (width 0.2) (layer "F.Cu") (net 8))
 (segment (start 115 93.75) (end 115 94.2348) (width 0.2) (layer "F.Cu") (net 31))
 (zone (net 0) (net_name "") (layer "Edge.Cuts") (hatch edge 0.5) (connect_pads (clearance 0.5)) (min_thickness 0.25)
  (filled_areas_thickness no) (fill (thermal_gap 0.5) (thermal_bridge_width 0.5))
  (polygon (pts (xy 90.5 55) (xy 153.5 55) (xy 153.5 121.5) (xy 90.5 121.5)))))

